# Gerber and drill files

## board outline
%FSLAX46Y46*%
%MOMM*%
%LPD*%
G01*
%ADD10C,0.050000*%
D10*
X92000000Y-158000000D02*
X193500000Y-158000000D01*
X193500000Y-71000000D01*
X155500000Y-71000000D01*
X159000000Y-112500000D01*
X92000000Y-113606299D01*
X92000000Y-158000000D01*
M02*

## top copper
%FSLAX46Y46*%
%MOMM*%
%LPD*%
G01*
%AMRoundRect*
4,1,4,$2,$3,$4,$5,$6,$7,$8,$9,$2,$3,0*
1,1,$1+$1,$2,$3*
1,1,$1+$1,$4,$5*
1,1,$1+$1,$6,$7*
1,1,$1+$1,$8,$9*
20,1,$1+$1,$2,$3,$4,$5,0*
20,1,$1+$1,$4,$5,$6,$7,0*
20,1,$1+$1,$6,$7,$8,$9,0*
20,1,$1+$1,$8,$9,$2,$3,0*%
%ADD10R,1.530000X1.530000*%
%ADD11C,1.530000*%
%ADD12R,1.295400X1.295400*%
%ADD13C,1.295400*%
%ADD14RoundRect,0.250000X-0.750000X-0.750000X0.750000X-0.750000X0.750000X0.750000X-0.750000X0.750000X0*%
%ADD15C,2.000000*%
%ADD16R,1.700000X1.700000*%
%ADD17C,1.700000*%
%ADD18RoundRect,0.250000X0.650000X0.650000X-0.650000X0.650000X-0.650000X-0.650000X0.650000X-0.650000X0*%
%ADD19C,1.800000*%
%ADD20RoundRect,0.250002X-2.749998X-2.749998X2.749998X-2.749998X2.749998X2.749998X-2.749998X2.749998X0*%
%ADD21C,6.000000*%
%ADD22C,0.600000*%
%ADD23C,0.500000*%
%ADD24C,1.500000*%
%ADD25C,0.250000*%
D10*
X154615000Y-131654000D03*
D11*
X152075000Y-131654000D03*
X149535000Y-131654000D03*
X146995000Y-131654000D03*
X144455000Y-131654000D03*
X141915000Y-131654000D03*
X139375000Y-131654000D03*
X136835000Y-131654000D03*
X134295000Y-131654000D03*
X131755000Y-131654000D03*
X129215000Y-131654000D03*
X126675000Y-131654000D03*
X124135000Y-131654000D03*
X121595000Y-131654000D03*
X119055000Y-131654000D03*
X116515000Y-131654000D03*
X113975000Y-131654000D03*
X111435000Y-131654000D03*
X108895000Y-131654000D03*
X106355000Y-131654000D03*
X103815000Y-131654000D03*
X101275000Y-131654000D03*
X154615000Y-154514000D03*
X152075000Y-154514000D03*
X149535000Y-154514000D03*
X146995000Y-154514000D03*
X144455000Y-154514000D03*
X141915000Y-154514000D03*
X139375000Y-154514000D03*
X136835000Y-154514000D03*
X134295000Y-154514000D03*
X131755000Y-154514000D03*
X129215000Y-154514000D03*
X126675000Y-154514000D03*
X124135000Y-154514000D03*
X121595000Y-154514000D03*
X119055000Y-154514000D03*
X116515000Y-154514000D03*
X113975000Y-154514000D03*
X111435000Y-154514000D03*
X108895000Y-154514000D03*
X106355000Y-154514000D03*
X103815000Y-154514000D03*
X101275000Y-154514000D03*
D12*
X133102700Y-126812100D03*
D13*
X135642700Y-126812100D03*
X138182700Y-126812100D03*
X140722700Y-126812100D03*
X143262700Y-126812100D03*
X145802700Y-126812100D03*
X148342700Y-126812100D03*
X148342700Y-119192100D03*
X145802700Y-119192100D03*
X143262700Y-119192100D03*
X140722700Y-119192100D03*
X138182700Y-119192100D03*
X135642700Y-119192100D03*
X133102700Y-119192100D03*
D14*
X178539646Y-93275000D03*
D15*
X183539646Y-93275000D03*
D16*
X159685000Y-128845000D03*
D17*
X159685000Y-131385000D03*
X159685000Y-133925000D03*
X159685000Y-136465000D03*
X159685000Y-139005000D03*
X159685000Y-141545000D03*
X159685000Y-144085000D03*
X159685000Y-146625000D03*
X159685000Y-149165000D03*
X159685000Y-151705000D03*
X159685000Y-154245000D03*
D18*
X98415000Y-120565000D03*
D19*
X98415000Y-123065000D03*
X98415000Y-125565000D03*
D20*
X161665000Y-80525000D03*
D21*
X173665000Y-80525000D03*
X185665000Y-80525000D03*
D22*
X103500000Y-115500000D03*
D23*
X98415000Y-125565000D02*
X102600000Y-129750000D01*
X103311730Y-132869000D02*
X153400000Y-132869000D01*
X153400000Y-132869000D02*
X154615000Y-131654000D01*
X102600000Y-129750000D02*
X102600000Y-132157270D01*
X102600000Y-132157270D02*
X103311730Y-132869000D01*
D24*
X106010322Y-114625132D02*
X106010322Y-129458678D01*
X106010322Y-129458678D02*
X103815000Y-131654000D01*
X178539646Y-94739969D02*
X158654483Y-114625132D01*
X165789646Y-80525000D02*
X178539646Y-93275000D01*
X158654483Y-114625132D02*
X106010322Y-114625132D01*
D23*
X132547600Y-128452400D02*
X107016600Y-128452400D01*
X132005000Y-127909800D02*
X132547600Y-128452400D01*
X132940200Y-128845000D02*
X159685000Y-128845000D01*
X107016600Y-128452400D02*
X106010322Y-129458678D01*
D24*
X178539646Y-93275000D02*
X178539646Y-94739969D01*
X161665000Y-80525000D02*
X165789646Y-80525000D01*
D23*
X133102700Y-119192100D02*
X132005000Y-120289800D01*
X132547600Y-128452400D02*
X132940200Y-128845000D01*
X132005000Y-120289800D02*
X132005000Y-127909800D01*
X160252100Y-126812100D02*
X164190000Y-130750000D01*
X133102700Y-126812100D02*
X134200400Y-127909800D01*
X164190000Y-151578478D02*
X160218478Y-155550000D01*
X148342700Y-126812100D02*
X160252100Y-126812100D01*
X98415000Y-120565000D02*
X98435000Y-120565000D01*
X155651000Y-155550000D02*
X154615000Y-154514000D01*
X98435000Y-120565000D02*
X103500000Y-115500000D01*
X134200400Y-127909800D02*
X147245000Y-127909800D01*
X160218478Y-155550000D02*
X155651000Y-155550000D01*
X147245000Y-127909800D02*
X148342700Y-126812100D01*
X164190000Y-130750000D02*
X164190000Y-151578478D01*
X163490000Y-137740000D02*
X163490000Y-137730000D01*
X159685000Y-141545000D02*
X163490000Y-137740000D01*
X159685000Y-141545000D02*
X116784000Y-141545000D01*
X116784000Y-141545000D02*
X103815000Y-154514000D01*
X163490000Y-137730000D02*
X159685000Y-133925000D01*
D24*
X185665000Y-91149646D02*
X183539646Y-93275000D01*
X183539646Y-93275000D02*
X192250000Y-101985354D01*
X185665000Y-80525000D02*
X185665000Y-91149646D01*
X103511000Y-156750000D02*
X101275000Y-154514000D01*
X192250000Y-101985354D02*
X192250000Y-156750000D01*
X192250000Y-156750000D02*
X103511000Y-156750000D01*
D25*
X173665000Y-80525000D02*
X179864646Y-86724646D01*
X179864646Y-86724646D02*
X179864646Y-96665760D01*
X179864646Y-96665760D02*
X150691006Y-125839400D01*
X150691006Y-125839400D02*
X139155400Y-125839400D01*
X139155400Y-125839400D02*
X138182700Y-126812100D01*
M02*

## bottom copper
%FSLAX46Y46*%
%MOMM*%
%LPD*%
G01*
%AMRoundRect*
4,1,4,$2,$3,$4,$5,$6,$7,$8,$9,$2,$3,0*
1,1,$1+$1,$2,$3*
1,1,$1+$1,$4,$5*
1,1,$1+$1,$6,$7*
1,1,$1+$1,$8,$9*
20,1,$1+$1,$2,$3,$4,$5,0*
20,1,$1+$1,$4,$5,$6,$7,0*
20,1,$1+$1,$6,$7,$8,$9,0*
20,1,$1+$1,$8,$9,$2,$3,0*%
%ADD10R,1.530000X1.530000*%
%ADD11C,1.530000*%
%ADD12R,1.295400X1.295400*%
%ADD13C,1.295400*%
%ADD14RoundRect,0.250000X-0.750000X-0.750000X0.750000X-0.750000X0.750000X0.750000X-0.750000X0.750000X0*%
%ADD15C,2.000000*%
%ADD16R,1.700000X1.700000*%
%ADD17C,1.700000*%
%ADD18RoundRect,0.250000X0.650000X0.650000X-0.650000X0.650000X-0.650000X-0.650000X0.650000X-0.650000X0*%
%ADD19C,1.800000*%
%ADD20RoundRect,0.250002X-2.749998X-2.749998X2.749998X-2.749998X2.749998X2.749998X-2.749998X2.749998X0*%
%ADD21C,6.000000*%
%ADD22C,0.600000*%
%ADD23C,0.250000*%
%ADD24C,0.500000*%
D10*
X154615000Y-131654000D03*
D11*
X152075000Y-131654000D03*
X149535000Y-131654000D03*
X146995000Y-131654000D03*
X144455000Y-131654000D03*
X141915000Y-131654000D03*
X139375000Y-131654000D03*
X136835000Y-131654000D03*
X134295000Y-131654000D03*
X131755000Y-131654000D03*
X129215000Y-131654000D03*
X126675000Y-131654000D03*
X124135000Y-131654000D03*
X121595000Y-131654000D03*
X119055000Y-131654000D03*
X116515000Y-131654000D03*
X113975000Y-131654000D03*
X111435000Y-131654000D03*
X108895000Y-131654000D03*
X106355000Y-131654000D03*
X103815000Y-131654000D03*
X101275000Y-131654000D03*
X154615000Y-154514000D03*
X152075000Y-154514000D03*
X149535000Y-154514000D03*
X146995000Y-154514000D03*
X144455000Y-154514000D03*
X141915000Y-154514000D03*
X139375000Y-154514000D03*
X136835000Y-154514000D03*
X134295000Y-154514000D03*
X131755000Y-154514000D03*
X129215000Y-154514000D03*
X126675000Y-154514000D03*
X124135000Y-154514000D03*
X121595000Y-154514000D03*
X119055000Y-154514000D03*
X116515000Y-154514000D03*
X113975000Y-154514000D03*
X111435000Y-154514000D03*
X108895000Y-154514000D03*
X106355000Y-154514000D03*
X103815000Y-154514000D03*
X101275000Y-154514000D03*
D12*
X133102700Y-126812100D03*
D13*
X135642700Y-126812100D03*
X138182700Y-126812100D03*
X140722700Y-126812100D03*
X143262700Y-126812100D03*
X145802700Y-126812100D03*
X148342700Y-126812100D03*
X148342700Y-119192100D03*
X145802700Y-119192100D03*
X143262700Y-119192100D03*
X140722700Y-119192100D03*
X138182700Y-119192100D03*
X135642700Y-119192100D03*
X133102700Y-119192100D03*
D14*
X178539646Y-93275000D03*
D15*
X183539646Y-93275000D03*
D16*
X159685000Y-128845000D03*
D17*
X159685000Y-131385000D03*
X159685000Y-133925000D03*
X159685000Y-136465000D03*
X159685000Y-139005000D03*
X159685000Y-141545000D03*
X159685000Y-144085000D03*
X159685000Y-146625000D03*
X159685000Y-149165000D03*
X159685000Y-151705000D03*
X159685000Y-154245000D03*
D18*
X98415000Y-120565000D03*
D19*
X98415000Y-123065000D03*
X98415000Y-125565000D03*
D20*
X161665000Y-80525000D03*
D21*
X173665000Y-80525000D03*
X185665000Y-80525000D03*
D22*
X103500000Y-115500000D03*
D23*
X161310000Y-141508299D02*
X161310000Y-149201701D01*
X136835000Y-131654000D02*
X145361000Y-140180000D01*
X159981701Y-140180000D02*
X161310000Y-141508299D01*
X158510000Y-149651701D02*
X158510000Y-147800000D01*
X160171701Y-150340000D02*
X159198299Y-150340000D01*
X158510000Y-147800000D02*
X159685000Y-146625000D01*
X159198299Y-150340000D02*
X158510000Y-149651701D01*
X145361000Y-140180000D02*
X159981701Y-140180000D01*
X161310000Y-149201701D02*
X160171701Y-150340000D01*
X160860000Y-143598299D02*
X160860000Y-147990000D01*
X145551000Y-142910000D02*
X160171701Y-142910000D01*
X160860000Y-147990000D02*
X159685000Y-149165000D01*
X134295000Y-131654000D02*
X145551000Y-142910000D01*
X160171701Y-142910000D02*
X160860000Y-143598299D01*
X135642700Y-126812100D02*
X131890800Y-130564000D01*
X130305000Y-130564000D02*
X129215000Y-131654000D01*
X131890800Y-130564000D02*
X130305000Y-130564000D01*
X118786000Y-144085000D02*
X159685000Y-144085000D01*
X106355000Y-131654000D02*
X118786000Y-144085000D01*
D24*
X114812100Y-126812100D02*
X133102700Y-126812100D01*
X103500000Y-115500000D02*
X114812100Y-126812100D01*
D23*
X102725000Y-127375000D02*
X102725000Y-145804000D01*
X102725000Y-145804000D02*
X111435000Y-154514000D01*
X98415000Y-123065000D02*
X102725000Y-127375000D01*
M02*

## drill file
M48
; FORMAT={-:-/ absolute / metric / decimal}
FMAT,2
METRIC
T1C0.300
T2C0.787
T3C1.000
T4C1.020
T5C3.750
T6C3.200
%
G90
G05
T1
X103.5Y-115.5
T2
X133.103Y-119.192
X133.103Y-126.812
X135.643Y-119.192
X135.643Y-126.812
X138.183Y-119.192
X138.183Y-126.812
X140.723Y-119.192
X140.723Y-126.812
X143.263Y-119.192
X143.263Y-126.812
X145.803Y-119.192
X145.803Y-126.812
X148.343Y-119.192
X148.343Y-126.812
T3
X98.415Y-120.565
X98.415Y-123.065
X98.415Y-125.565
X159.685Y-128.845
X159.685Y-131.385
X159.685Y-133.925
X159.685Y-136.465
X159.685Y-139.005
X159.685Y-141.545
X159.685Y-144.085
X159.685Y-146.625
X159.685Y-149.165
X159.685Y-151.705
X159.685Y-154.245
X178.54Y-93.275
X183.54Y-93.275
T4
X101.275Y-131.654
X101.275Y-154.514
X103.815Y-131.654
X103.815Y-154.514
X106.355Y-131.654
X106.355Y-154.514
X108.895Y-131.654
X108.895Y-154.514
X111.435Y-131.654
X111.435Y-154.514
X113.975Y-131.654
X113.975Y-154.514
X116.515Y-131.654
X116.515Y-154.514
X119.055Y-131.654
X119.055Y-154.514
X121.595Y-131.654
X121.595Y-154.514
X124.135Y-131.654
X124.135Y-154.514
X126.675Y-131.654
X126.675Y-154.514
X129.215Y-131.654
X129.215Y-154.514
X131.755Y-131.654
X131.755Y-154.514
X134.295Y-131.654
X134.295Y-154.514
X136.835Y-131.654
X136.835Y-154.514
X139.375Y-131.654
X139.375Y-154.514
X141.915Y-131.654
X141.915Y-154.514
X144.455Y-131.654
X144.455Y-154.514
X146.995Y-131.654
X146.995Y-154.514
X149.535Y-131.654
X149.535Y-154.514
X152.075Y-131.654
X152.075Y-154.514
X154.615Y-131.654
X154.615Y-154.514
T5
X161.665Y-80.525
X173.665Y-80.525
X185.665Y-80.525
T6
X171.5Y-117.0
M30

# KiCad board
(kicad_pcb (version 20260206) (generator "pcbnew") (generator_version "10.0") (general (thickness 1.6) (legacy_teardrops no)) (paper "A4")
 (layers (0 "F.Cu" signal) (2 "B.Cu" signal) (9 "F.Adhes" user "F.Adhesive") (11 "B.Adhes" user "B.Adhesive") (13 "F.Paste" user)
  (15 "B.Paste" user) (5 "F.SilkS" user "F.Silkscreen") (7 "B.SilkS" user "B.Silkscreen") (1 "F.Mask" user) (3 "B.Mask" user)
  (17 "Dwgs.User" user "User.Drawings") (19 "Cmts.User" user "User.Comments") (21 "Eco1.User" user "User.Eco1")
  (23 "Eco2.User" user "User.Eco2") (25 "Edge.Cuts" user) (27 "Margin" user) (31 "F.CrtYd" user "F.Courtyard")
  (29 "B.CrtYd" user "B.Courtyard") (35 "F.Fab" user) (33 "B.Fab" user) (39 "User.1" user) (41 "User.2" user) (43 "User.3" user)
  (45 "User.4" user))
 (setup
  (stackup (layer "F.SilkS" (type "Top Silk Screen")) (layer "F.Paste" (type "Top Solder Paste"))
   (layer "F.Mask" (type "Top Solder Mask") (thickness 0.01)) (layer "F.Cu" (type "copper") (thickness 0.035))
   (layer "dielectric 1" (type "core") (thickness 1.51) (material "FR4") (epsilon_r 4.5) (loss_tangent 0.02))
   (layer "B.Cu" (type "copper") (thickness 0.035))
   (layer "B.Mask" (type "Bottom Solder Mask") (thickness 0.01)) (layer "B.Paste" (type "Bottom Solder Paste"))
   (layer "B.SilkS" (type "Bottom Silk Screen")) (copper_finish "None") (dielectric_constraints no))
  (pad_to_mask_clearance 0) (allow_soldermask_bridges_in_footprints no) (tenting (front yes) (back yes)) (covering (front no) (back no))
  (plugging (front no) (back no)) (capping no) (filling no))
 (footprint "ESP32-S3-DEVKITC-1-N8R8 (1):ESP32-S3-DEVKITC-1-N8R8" (layer "F.Cu") (at 124.645 143.084 -90)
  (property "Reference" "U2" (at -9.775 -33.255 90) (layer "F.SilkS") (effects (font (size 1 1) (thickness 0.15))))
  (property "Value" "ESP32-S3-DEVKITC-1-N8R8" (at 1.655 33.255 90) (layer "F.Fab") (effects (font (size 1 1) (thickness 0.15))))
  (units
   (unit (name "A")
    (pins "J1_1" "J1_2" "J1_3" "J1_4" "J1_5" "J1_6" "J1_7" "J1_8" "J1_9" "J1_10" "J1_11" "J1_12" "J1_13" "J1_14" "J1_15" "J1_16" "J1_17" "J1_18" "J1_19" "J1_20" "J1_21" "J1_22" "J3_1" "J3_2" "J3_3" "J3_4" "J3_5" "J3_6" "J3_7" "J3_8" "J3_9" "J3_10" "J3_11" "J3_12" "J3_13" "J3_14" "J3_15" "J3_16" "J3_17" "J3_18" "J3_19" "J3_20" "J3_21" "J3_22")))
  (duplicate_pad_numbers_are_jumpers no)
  (pad "J1_1" thru_hole rect (at -11.43 -29.97 270) (size 1.53 1.53) (drill 1.02) (layers "*.Cu" "*.Mask") (remove_unused_layers no)
   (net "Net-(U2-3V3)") (solder_mask_margin 0.102))
  (pad "J1_2" thru_hole circle (at -11.43 -27.43 270) (size 1.53 1.53) (drill 1.02) (layers "*.Cu" "*.Mask") (remove_unused_layers no)
   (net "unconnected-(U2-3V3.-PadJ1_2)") (solder_mask_margin 0.102))
  (pad "J1_3" thru_hole circle (at -11.43 -24.89 270) (size 1.53 1.53) (drill 1.02) (layers "*.Cu" "*.Mask") (remove_unused_layers no)
   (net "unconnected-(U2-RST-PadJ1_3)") (solder_mask_margin 0.102))
  (pad "J1_4" thru_hole circle (at -11.43 -22.35 270) (size 1.53 1.53) (drill 1.02) (layers "*.Cu" "*.Mask") (remove_unused_layers no)
   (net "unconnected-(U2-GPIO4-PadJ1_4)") (solder_mask_margin 0.102))
  (pad "J1_5" thru_hole circle (at -11.43 -19.81 270) (size 1.53 1.53) (drill 1.02) (layers "*.Cu" "*.Mask") (remove_unused_layers no)
   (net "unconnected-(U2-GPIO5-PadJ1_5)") (solder_mask_margin 0.102))
  (pad "J1_6" thru_hole circle (at -11.43 -17.27 270) (size 1.53 1.53) (drill 1.02) (layers "*.Cu" "*.Mask") (remove_unused_layers no)
   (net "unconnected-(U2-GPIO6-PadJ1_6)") (solder_mask_margin 0.102))
  (pad "J1_7" thru_hole circle (at -11.43 -14.73 270) (size 1.53 1.53) (drill 1.02) (layers "*.Cu" "*.Mask") (remove_unused_layers no)
   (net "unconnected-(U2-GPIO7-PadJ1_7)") (solder_mask_margin 0.102))
  (pad "J1_8" thru_hole circle (at -11.43 -12.19 270) (size 1.53 1.53) (drill 1.02) (layers "*.Cu" "*.Mask") (remove_unused_layers no)
   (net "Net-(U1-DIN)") (solder_mask_margin 0.102))
  (pad "J1_9" thru_hole circle (at -11.43 -9.65 270) (size 1.53 1.53) (drill 1.02) (layers "*.Cu" "*.Mask") (remove_unused_layers no)
   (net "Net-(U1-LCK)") (solder_mask_margin 0.102))
  (pad "J1_10" thru_hole circle (at -11.43 -7.11 270) (size 1.53 1.53) (drill 1.02) (layers "*.Cu" "*.Mask") (remove_unused_layers no)
   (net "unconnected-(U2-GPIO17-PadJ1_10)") (solder_mask_margin 0.102))
  (pad "J1_11" thru_hole circle (at -11.43 -4.57 270) (size 1.53 1.53) (drill 1.02) (layers "*.Cu" "*.Mask") (remove_unused_layers no)
   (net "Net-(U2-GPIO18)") (solder_mask_margin 0.102))
  (pad "J1_12" thru_hole circle (at -11.43 -2.03 270) (size 1.53 1.53) (drill 1.02) (layers "*.Cu" "*.Mask") (remove_unused_layers no)
   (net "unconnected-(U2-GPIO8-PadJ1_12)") (solder_mask_margin 0.102))
  (pad "J1_13" thru_hole circle (at -11.43 0.51 270) (size 1.53 1.53) (drill 1.02) (layers "*.Cu" "*.Mask") (remove_unused_layers no)
   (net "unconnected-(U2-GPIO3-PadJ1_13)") (solder_mask_margin 0.102))
  (pad "J1_14" thru_hole circle (at -11.43 3.05 270) (size 1.53 1.53) (drill 1.02) (layers "*.Cu" "*.Mask") (remove_unused_layers no)
   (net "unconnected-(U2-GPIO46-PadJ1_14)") (solder_mask_margin 0.102))
  (pad "J1_15" thru_hole circle (at -11.43 5.59 270) (size 1.53 1.53) (drill 1.02) (layers "*.Cu" "*.Mask") (remove_unused_layers no)
   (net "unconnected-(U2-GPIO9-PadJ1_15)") (solder_mask_margin 0.102))
  (pad "J1_16" thru_hole circle (at -11.43 8.13 270) (size 1.53 1.53) (drill 1.02) (layers "*.Cu" "*.Mask") (remove_unused_layers no)
   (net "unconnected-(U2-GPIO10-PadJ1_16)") (solder_mask_margin 0.102))
  (pad "J1_17" thru_hole circle (at -11.43 10.67 270) (size 1.53 1.53) (drill 1.02) (layers "*.Cu" "*.Mask") (remove_unused_layers no)
   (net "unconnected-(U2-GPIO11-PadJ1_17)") (solder_mask_margin 0.102))
  (pad "J1_18" thru_hole circle (at -11.43 13.21 270) (size 1.53 1.53) (drill 1.02) (layers "*.Cu" "*.Mask") (remove_unused_layers no)
   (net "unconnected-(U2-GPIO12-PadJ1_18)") (solder_mask_margin 0.102))
  (pad "J1_19" thru_hole circle (at -11.43 15.75 270) (size 1.53 1.53) (drill 1.02) (layers "*.Cu" "*.Mask") (remove_unused_layers no)
   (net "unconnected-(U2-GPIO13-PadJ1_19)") (solder_mask_margin 0.102))
  (pad "J1_20" thru_hole circle (at -11.43 18.29 270) (size 1.53 1.53) (drill 1.02) (layers "*.Cu" "*.Mask") (remove_unused_layers no)
   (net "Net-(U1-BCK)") (solder_mask_margin 0.102))
  (pad "J1_21" thru_hole circle (at -11.43 20.83 270) (size 1.53 1.53) (drill 1.02) (layers "*.Cu" "*.Mask") (remove_unused_layers no)
   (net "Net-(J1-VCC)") (solder_mask_margin 0.102))
  (pad "J1_22" thru_hole circle (at -11.43 23.37 270) (size 1.53 1.53) (drill 1.02) (layers "*.Cu" "*.Mask") (remove_unused_layers no)
   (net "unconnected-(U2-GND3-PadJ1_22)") (solder_mask_margin 0.102))
  (pad "J3_1" thru_hole circle (at 11.43 -29.97 270) (size 1.53 1.53) (drill 1.02) (layers "*.Cu" "*.Mask") (remove_unused_layers no)
   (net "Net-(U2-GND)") (solder_mask_margin 0.102))
  (pad "J3_2" thru_hole circle (at 11.43 -27.43 270) (size 1.53 1.53) (drill 1.02) (layers "*.Cu" "*.Mask") (remove_unused_layers no)
   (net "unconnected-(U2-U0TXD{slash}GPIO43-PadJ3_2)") (solder_mask_margin 0.102))
  (pad "J3_3" thru_hole circle (at 11.43 -24.89 270) (size 1.53 1.53) (drill 1.02) (layers "*.Cu" "*.Mask") (remove_unused_layers no)
   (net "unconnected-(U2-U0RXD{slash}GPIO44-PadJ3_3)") (solder_mask_margin 0.102))
  (pad "J3_4" thru_hole circle (at 11.43 -22.35 270) (size 1.53 1.53) (drill 1.02) (layers "*.Cu" "*.Mask") (remove_unused_layers no)
   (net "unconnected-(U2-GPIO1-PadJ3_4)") (solder_mask_margin 0.102))
  (pad "J3_5" thru_hole circle (at 11.43 -19.81 270) (size 1.53 1.53) (drill 1.02) (layers "*.Cu" "*.Mask") (remove_unused_layers no)
   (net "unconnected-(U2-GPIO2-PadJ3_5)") (solder_mask_margin 0.102))
  (pad "J3_6" thru_hole circle (at 11.43 -17.27 270) (size 1.53 1.53) (drill 1.02) (layers "*.Cu" "*.Mask") (remove_unused_layers no)
   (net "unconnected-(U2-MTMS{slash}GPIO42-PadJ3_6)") (solder_mask_margin 0.102))
  (pad "J3_7" thru_hole circle (at 11.43 -14.73 270) (size 1.53 1.53) (drill 1.02) (layers "*.Cu" "*.Mask") (remove_unused_layers no)
   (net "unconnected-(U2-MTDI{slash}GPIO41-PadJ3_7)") (solder_mask_margin 0.102))
  (pad "J3_8" thru_hole circle (at 11.43 -12.19 270) (size 1.53 1.53) (drill 1.02) (layers "*.Cu" "*.Mask") (remove_unused_layers no)
   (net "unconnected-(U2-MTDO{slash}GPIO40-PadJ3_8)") (solder_mask_margin 0.102))
  (pad "J3_9" thru_hole circle (at 11.43 -9.65 270) (size 1.53 1.53) (drill 1.02) (layers "*.Cu" "*.Mask") (remove_unused_layers no)
   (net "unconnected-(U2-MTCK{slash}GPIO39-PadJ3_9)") (solder_mask_margin 0.102))
  (pad "J3_10" thru_hole circle (at 11.43 -7.11 270) (size 1.53 1.53) (drill 1.02) (layers "*.Cu" "*.Mask") (remove_unused_layers no)
   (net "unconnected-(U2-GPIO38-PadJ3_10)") (solder_mask_margin 0.102))
  (pad "J3_11" thru_hole circle (at 11.43 -4.57 270) (size 1.53 1.53) (drill 1.02) (layers "*.Cu" "*.Mask") (remove_unused_layers no)
   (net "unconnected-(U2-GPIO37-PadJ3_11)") (solder_mask_margin 0.102))
  (pad "J3_12" thru_hole circle (at 11.43 -2.03 270) (size 1.53 1.53) (drill 1.02) (layers "*.Cu" "*.Mask") (remove_unused_layers no)
   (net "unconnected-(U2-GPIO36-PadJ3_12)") (solder_mask_margin 0.102))
  (pad "J3_13" thru_hole circle (at 11.43 0.51 270) (size 1.53 1.53) (drill 1.02) (layers "*.Cu" "*.Mask") (remove_unused_layers no)
   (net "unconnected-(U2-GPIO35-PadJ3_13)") (solder_mask_margin 0.102))
  (pad "J3_14" thru_hole circle (at 11.43 3.05 270) (size 1.53 1.53) (drill 1.02) (layers "*.Cu" "*.Mask") (remove_unused_layers no)
   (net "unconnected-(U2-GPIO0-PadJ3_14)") (solder_mask_margin 0.102))
  (pad "J3_15" thru_hole circle (at 11.43 5.59 270) (size 1.53 1.53) (drill 1.02) (layers "*.Cu" "*.Mask") (remove_unused_layers no)
   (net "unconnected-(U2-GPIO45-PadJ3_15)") (solder_mask_margin 0.102))
  (pad "J3_16" thru_hole circle (at 11.43 8.13 270) (size 1.53 1.53) (drill 1.02) (layers "*.Cu" "*.Mask") (remove_unused_layers no)
   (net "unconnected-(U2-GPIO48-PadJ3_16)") (solder_mask_margin 0.102))
  (pad "J3_17" thru_hole circle (at 11.43 10.67 270) (size 1.53 1.53) (drill 1.02) (layers "*.Cu" "*.Mask") (remove_unused_layers no)
   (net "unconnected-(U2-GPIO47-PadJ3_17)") (solder_mask_margin 0.102))
  (pad "J3_18" thru_hole circle (at 11.43 13.21 270) (size 1.53 1.53) (drill 1.02) (layers "*.Cu" "*.Mask") (remove_unused_layers no)
   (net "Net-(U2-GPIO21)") (solder_mask_margin 0.102))
  (pad "J3_19" thru_hole circle (at 11.43 15.75 270) (size 1.53 1.53) (drill 1.02) (layers "*.Cu" "*.Mask") (remove_unused_layers no)
   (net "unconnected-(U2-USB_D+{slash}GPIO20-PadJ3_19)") (solder_mask_margin 0.102))
  (pad "J3_20" thru_hole circle (at 11.43 18.29 270) (size 1.53 1.53) (drill 1.02) (layers "*.Cu" "*.Mask") (remove_unused_layers no)
   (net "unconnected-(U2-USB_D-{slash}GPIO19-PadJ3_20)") (solder_mask_margin 0.102))
  (pad "J3_21" thru_hole circle (at 11.43 20.83 270) (size 1.53 1.53) (drill 1.02) (layers "*.Cu" "*.Mask") (remove_unused_layers no)
   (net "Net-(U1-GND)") (solder_mask_margin 0.102))
  (pad "J3_22" thru_hole circle (at 11.43 23.37 270) (size 1.53 1.53) (drill 1.02) (layers "*.Cu" "*.Mask") (remove_unused_layers no)
   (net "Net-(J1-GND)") (solder_mask_margin 0.102)))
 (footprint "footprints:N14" (layer "F.Cu") (at 148.3427 119.1921 90)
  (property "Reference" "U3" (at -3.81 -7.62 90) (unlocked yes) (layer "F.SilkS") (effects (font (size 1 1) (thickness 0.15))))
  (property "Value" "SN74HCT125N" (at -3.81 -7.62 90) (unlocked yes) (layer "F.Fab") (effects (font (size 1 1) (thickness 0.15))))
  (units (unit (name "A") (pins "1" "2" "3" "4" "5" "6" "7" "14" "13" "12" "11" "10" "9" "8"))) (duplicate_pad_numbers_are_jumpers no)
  (pad "1" thru_hole rect (at -7.62 -15.24 90) (size 1.2954 1.2954) (drill 0.7874) (layers "*.Cu" "*.Mask") (remove_unused_layers no)
   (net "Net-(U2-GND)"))
  (pad "2" thru_hole circle (at -7.62 -12.7 90) (size 1.2954 1.2954) (drill 0.7874) (layers "*.Cu" "*.Mask") (remove_unused_layers no)
   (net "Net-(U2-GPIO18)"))
  (pad "3" thru_hole circle (at -7.62 -10.16 90) (size 1.2954 1.2954) (drill 0.7874) (layers "*.Cu" "*.Mask") (remove_unused_layers no)
   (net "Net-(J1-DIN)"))
  (pad "4" thru_hole circle (at -7.62 -7.62 90) (size 1.2954 1.2954) (drill 0.7874) (layers "*.Cu" "*.Mask") (remove_unused_layers no)
   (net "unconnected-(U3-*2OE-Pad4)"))
  (pad "5" thru_hole circle (at -7.62 -5.08 90) (size 1.2954 1.2954) (drill 0.7874) (layers "*.Cu" "*.Mask") (remove_unused_layers no)
   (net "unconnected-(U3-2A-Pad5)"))
  (pad "6" thru_hole circle (at -7.62 -2.54 90) (size 1.2954 1.2954) (drill 0.7874) (layers "*.Cu" "*.Mask") (remove_unused_layers no)
   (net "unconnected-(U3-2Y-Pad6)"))
  (pad "7" thru_hole circle (at -7.62 0 90) (size 1.2954 1.2954) (drill 0.7874) (layers "*.Cu" "*.Mask") (remove_unused_layers no)
   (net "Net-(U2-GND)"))
  (pad "8" thru_hole circle (at 0 0 90) (size 1.2954 1.2954) (drill 0.7874) (layers "*.Cu" "*.Mask") (remove_unused_layers no)
   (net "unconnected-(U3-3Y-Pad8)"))
  (pad "9" thru_hole circle (at 0 -2.54 90) (size 1.2954 1.2954) (drill 0.7874) (layers "*.Cu" "*.Mask") (remove_unused_layers no)
   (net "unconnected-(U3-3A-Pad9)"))
  (pad "10" thru_hole circle (at 0 -5.08 90) (size 1.2954 1.2954) (drill 0.7874) (layers "*.Cu" "*.Mask") (remove_unused_layers no)
   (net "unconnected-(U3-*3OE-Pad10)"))
  (pad "11" thru_hole circle (at 0 -7.62 90) (size 1.2954 1.2954) (drill 0.7874) (layers "*.Cu" "*.Mask") (remove_unused_layers no)
   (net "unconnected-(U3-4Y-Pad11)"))
  (pad "12" thru_hole circle (at 0 -10.16 90) (size 1.2954 1.2954) (drill 0.7874) (layers "*.Cu" "*.Mask") (remove_unused_layers no)
   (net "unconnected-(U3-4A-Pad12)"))
  (pad "13" thru_hole circle (at 0 -12.7 90) (size 1.2954 1.2954) (drill 0.7874) (layers "*.Cu" "*.Mask") (remove_unused_layers no)
   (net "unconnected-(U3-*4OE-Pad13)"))
  (pad "14" thru_hole circle (at 0 -15.24 90) (size 1.2954 1.2954) (drill 0.7874) (layers "*.Cu" "*.Mask") (remove_unused_layers no)
   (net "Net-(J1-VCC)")))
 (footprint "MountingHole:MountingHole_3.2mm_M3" (layer "F.Cu") (at 171.5 117)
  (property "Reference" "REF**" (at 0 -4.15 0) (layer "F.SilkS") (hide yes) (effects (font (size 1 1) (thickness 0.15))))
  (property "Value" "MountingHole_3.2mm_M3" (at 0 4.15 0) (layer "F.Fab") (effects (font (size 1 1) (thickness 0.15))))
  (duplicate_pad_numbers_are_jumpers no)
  (pad "" np_thru_hole circle (at 0 0) (size 3.2 3.2) (drill 3.2) (layers "*.Cu" "*.Mask")))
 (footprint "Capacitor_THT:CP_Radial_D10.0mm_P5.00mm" (layer "F.Cu") (at 178.539646 93.275)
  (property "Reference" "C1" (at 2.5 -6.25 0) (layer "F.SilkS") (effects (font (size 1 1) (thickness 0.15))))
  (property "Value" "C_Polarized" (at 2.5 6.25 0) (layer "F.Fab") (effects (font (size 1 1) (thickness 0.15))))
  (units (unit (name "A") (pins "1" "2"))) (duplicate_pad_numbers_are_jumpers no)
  (pad "1" thru_hole roundrect (at 0 0) (size 2 2) (drill 1) (layers "*.Cu" "*.Mask") (remove_unused_layers no) (roundrect_rratio 0.125)
   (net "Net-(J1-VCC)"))
  (pad "2" thru_hole circle (at 5 0) (size 2 2) (drill 1) (layers "*.Cu" "*.Mask") (remove_unused_layers no) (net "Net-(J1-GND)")))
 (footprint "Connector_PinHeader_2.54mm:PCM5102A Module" (layer "F.Cu") (at 159.685 128.845)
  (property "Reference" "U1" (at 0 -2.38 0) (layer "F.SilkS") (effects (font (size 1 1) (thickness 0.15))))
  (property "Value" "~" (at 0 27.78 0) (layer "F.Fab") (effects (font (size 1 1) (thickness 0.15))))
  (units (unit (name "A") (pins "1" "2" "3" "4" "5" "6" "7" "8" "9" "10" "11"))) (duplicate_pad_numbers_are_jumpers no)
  (pad "1" thru_hole rect (at 0 0) (size 1.7 1.7) (drill 1) (layers "*.Cu" "*.Mask") (remove_unused_layers no) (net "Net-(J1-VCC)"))
  (pad "2" thru_hole circle (at 0 2.54) (size 1.7 1.7) (drill 1) (layers "*.Cu" "*.Mask") (remove_unused_layers no)
   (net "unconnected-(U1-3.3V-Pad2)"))
  (pad "3" thru_hole circle (at 0 5.08) (size 1.7 1.7) (drill 1) (layers "*.Cu" "*.Mask") (remove_unused_layers no) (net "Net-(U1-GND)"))
  (pad "4" thru_hole circle (at 0 7.62) (size 1.7 1.7) (drill 1) (layers "*.Cu" "*.Mask") (remove_unused_layers no)
   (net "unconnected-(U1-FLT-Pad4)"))
  (pad "5" thru_hole circle (at 0 10.16) (size 1.7 1.7) (drill 1) (layers "*.Cu" "*.Mask") (remove_unused_layers no)
   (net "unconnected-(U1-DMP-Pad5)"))
  (pad "6" thru_hole circle (at 0 12.7) (size 1.7 1.7) (drill 1) (layers "*.Cu" "*.Mask") (remove_unused_layers no) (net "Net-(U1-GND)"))
  (pad "7" thru_hole circle (at 0 15.24) (size 1.7 1.7) (drill 1) (layers "*.Cu" "*.Mask") (remove_unused_layers no) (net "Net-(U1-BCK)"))
  (pad "8" thru_hole circle (at 0 17.78) (size 1.7 1.7) (drill 1) (layers "*.Cu" "*.Mask") (remove_unused_layers no) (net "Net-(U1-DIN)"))
  (pad "9" thru_hole circle (at 0 20.32) (size 1.7 1.7) (drill 1) (layers "*.Cu" "*.Mask") (remove_unused_layers no) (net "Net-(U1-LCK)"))
  (pad "10" thru_hole circle (at 0 22.86) (size 1.7 1.7) (drill 1) (layers "*.Cu" "*.Mask") (remove_unused_layers no)
   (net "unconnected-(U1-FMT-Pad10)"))
  (pad "11" thru_hole circle (at 0 25.4) (size 1.7 1.7) (drill 1) (layers "*.Cu" "*.Mask") (remove_unused_layers no)
   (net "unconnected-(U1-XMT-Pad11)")))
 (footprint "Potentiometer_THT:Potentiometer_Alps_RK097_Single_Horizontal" (layer "F.Cu") (at 98.415 120.565)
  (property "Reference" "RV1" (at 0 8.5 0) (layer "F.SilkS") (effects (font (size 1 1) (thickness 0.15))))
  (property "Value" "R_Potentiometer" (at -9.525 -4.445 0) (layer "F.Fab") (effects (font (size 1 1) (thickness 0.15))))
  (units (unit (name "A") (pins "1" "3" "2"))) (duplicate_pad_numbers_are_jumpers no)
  (pad "1" thru_hole roundrect (at 0 0 180) (size 1.8 1.8) (drill 1) (layers "*.Cu" "*.Mask") (remove_unused_layers no)
   (roundrect_rratio 0.1388888889) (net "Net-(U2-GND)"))
  (pad "2" thru_hole circle (at 0 2.5 180) (size 1.8 1.8) (drill 1) (layers "*.Cu" "*.Mask") (remove_unused_layers no)
   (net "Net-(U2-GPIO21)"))
  (pad "3" thru_hole circle (at 0 5 180) (size 1.8 1.8) (drill 1) (layers "*.Cu" "*.Mask") (remove_unused_layers no) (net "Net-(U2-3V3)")))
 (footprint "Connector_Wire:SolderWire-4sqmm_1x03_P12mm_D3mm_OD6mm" (layer "F.Cu") (at 161.665 80.525)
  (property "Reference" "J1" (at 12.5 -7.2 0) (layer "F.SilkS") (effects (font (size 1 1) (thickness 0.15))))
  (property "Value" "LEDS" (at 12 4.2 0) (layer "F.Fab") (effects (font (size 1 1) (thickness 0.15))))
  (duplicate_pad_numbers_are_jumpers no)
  (pad "1" thru_hole roundrect (at 0 0) (size 6 6) (drill 3.75) (layers "*.Cu" "*.Mask") (remove_unused_layers no)
   (roundrect_rratio 0.041667) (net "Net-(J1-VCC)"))
  (pad "2" thru_hole circle (at 12 0) (size 6 6) (drill 3.75) (layers "*.Cu" "*.Mask") (remove_unused_layers no) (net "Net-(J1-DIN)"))
  (pad "3" thru_hole circle (at 24 0) (size 6 6) (drill 3.75) (layers "*.Cu" "*.Mask") (remove_unused_layers no) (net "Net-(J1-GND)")))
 (gr_poly
  (pts (xy 92 158) (xy 193.5 158) (xy 193.5 71) (xy 155.5 71) (xy 159 112.5) (xy 92 113.606299)) (stroke (width 0.05) (type solid))
  (fill no) (layer "Edge.Cuts"))
 (segment (start 98.415 125.565) (end 102.6 129.75) (width 0.5) (layer "F.Cu") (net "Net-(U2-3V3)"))
 (segment (start 103.31173 132.869) (end 153.4 132.869) (width 0.5) (layer "F.Cu") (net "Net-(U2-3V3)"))
 (segment (start 153.4 132.869) (end 154.615 131.654) (width 0.5) (layer "F.Cu") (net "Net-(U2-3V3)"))
 (segment (start 102.6 129.75) (end 102.6 132.15727) (width 0.5) (layer "F.Cu") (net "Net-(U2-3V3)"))
 (segment (start 102.6 132.15727) (end 103.31173 132.869) (width 0.5) (layer "F.Cu") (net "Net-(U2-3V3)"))
 (segment (start 161.31 141.508299) (end 161.31 149.201701) (width 0.25) (layer "B.Cu") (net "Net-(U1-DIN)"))
 (segment (start 136.835 131.654) (end 145.361 140.18) (width 0.25) (layer "B.Cu") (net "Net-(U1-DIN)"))
 (segment (start 159.981701 140.18) (end 161.31 141.508299) (width 0.25) (layer "B.Cu") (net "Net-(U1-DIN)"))
 (segment (start 158.51 149.651701) (end 158.51 147.8) (width 0.25) (layer "B.Cu") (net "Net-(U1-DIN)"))
 (segment (start 160.171701 150.34) (end 159.198299 150.34) (width 0.25) (layer "B.Cu") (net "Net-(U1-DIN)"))
 (segment (start 158.51 147.8) (end 159.685 146.625) (width 0.25) (layer "B.Cu") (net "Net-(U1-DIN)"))
 (segment (start 159.198299 150.34) (end 158.51 149.651701) (width 0.25) (layer "B.Cu") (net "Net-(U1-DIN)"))
 (segment (start 145.361 140.18) (end 159.981701 140.18) (width 0.25) (layer "B.Cu") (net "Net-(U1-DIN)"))
 (segment (start 161.31 149.201701) (end 160.171701 150.34) (width 0.25) (layer "B.Cu") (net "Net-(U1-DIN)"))
 (segment (start 160.86 143.598299) (end 160.86 147.99) (width 0.25) (layer "B.Cu") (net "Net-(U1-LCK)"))
 (segment (start 145.551 142.91) (end 160.171701 142.91) (width 0.25) (layer "B.Cu") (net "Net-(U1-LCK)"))
 (segment (start 160.86 147.99) (end 159.685 149.165) (width 0.25) (layer "B.Cu") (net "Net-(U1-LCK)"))
 (segment (start 134.295 131.654) (end 145.551 142.91) (width 0.25) (layer "B.Cu") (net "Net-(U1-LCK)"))
 (segment (start 160.171701 142.91) (end 160.86 143.598299) (width 0.25) (layer "B.Cu") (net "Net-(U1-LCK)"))
 (segment (start 135.6427 126.8121) (end 131.8908 130.564) (width 0.25) (layer "B.Cu") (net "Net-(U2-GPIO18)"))
 (segment (start 130.305 130.564) (end 129.215 131.654) (width 0.25) (layer "B.Cu") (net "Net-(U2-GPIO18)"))
 (segment (start 131.8908 130.564) (end 130.305 130.564) (width 0.25) (layer "B.Cu") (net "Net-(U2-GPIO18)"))
 (segment (start 118.786 144.085) (end 159.685 144.085) (width 0.25) (layer "B.Cu") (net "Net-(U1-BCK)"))
 (segment (start 106.355 131.654) (end 118.786 144.085) (width 0.25) (layer "B.Cu") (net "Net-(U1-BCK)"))
 (segment (start 106.010322 114.625132) (end 106.010322 129.458678) (width 1.5) (layer "F.Cu") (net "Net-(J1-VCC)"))
 (segment (start 106.010322 129.458678) (end 103.815 131.654) (width 1.5) (layer "F.Cu") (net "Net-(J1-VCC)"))
 (segment (start 178.539646 94.739969) (end 158.654483 114.625132) (width 1.5) (layer "F.Cu") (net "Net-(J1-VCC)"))
 (segment (start 165.789646 80.525) (end 178.539646 93.275) (width 1.5) (layer "F.Cu") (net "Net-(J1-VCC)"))
 (segment (start 158.654483 114.625132) (end 106.010322 114.625132) (width 1.5) (layer "F.Cu") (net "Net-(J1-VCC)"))
 (segment (start 132.5476 128.4524) (end 107.0166 128.4524) (width 0.5) (layer "F.Cu") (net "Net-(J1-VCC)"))
 (segment (start 132.005 127.9098) (end 132.5476 128.4524) (width 0.5) (layer "F.Cu") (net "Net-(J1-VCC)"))
 (segment (start 132.9402 128.845) (end 159.685 128.845) (width 0.5) (layer "F.Cu") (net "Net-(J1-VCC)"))
 (segment (start 107.0166 128.4524) (end 106.010322 129.458678) (width 0.5) (layer "F.Cu") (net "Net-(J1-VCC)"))
 (segment (start 178.539646 93.275) (end 178.539646 94.739969) (width 1.5) (layer "F.Cu") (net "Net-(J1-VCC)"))
 (segment (start 161.665 80.525) (end 165.789646 80.525) (width 1.5) (layer "F.Cu") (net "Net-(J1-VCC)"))
 (segment (start 133.1027 119.1921) (end 132.005 120.2898) (width 0.5) (layer "F.Cu") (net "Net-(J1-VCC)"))
 (segment (start 132.5476 128.4524) (end 132.9402 128.845) (width 0.5) (layer "F.Cu") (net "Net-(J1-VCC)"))
 (segment (start 132.005 120.2898) (end 132.005 127.9098) (width 0.5) (layer "F.Cu") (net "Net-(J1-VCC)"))
 (segment (start 160.2521 126.8121) (end 164.19 130.75) (width 0.5) (layer "F.Cu") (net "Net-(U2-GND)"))
 (segment (start 133.1027 126.8121) (end 134.2004 127.9098) (width 0.5) (layer "F.Cu") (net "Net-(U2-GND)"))
 (segment (start 164.19 151.578478) (end 160.218478 155.55) (width 0.5) (layer "F.Cu") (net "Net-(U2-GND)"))
 (segment (start 148.3427 126.8121) (end 160.2521 126.8121) (width 0.5) (layer "F.Cu") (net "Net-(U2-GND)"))
 (segment (start 98.415 120.565) (end 98.435 120.565) (width 0.5) (layer "F.Cu") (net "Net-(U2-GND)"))
 (segment (start 155.651 155.55) (end 154.615 154.514) (width 0.5) (layer "F.Cu") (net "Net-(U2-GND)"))
 (segment (start 98.435 120.565) (end 103.5 115.5) (width 0.5) (layer "F.Cu") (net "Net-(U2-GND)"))
 (segment (start 134.2004 127.9098) (end 147.245 127.9098) (width 0.5) (layer "F.Cu") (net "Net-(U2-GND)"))
 (segment (start 160.218478 155.55) (end 155.651 155.55) (width 0.5) (layer "F.Cu") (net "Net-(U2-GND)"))
 (segment (start 147.245 127.9098) (end 148.3427 126.8121) (width 0.5) (layer "F.Cu") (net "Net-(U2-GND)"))
 (segment (start 164.19 130.75) (end 164.19 151.578478) (width 0.5) (layer "F.Cu") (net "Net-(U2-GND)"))
 (via (at 103.5 115.5) (size 0.6) (drill 0.3) (layers "F.Cu" "B.Cu") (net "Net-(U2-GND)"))
 (segment (start 114.8121 126.8121) (end 133.1027 126.8121) (width 0.5) (layer "B.Cu") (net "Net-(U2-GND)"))
 (segment (start 103.5 115.5) (end 114.8121 126.8121) (width 0.5) (layer "B.Cu") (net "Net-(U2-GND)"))
 (segment (start 102.725 127.375) (end 102.725 145.804) (width 0.25) (layer "B.Cu") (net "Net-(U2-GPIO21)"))
 (segment (start 102.725 145.804) (end 111.435 154.514) (width 0.25) (layer "B.Cu") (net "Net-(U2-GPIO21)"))
 (segment (start 98.415 123.065) (end 102.725 127.375) (width 0.25) (layer "B.Cu") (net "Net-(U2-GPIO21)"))
 (segment (start 163.49 137.74) (end 163.49 137.73) (width 0.5) (layer "F.Cu") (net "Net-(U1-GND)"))
 (segment (start 159.685 141.545) (end 163.49 137.74) (width 0.5) (layer "F.Cu") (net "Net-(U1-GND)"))
 (segment (start 159.685 141.545) (end 116.784 141.545) (width 0.5) (layer "F.Cu") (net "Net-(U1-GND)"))
 (segment (start 116.784 141.545) (end 103.815 154.514) (width 0.5) (layer "F.Cu") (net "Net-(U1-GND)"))
 (segment (start 163.49 137.73) (end 159.685 133.925) (width 0.5) (layer "F.Cu") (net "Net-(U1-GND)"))
 (segment (start 185.665 91.149646) (end 183.539646 93.275) (width 1.5) (layer "F.Cu") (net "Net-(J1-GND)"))
 (segment (start 183.539646 93.275) (end 192.25 101.985354) (width 1.5) (layer "F.Cu") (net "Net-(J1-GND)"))
 (segment (start 185.665 80.525) (end 185.665 91.149646) (width 1.5) (layer "F.Cu") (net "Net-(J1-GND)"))
 (segment (start 103.511 156.75) (end 101.275 154.514) (width 1.5) (layer "F.Cu") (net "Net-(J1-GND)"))
 (segment (start 192.25 101.985354) (end 192.25 156.75) (width 1.5) (layer "F.Cu") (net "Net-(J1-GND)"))
 (segment (start 192.25 156.75) (end 103.511 156.75) (width 1.5) (layer "F.Cu") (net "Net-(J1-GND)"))
 (segment (start 173.665 80.525) (end 179.864646 86.724646) (width 0.25) (layer "F.Cu") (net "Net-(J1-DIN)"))
 (segment (start 179.864646 86.724646) (end 179.864646 96.66576) (width 0.25) (layer "F.Cu") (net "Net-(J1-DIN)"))
 (segment (start 179.864646 96.66576) (end 150.691006 125.8394) (width 0.25) (layer "F.Cu") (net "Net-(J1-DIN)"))
 (segment (start 150.691006 125.8394) (end 139.1554 125.8394) (width 0.25) (layer "F.Cu") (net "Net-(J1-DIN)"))
 (segment (start 139.1554 125.8394) (end 138.1827 126.8121) (width 0.25) (layer "F.Cu") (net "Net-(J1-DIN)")))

